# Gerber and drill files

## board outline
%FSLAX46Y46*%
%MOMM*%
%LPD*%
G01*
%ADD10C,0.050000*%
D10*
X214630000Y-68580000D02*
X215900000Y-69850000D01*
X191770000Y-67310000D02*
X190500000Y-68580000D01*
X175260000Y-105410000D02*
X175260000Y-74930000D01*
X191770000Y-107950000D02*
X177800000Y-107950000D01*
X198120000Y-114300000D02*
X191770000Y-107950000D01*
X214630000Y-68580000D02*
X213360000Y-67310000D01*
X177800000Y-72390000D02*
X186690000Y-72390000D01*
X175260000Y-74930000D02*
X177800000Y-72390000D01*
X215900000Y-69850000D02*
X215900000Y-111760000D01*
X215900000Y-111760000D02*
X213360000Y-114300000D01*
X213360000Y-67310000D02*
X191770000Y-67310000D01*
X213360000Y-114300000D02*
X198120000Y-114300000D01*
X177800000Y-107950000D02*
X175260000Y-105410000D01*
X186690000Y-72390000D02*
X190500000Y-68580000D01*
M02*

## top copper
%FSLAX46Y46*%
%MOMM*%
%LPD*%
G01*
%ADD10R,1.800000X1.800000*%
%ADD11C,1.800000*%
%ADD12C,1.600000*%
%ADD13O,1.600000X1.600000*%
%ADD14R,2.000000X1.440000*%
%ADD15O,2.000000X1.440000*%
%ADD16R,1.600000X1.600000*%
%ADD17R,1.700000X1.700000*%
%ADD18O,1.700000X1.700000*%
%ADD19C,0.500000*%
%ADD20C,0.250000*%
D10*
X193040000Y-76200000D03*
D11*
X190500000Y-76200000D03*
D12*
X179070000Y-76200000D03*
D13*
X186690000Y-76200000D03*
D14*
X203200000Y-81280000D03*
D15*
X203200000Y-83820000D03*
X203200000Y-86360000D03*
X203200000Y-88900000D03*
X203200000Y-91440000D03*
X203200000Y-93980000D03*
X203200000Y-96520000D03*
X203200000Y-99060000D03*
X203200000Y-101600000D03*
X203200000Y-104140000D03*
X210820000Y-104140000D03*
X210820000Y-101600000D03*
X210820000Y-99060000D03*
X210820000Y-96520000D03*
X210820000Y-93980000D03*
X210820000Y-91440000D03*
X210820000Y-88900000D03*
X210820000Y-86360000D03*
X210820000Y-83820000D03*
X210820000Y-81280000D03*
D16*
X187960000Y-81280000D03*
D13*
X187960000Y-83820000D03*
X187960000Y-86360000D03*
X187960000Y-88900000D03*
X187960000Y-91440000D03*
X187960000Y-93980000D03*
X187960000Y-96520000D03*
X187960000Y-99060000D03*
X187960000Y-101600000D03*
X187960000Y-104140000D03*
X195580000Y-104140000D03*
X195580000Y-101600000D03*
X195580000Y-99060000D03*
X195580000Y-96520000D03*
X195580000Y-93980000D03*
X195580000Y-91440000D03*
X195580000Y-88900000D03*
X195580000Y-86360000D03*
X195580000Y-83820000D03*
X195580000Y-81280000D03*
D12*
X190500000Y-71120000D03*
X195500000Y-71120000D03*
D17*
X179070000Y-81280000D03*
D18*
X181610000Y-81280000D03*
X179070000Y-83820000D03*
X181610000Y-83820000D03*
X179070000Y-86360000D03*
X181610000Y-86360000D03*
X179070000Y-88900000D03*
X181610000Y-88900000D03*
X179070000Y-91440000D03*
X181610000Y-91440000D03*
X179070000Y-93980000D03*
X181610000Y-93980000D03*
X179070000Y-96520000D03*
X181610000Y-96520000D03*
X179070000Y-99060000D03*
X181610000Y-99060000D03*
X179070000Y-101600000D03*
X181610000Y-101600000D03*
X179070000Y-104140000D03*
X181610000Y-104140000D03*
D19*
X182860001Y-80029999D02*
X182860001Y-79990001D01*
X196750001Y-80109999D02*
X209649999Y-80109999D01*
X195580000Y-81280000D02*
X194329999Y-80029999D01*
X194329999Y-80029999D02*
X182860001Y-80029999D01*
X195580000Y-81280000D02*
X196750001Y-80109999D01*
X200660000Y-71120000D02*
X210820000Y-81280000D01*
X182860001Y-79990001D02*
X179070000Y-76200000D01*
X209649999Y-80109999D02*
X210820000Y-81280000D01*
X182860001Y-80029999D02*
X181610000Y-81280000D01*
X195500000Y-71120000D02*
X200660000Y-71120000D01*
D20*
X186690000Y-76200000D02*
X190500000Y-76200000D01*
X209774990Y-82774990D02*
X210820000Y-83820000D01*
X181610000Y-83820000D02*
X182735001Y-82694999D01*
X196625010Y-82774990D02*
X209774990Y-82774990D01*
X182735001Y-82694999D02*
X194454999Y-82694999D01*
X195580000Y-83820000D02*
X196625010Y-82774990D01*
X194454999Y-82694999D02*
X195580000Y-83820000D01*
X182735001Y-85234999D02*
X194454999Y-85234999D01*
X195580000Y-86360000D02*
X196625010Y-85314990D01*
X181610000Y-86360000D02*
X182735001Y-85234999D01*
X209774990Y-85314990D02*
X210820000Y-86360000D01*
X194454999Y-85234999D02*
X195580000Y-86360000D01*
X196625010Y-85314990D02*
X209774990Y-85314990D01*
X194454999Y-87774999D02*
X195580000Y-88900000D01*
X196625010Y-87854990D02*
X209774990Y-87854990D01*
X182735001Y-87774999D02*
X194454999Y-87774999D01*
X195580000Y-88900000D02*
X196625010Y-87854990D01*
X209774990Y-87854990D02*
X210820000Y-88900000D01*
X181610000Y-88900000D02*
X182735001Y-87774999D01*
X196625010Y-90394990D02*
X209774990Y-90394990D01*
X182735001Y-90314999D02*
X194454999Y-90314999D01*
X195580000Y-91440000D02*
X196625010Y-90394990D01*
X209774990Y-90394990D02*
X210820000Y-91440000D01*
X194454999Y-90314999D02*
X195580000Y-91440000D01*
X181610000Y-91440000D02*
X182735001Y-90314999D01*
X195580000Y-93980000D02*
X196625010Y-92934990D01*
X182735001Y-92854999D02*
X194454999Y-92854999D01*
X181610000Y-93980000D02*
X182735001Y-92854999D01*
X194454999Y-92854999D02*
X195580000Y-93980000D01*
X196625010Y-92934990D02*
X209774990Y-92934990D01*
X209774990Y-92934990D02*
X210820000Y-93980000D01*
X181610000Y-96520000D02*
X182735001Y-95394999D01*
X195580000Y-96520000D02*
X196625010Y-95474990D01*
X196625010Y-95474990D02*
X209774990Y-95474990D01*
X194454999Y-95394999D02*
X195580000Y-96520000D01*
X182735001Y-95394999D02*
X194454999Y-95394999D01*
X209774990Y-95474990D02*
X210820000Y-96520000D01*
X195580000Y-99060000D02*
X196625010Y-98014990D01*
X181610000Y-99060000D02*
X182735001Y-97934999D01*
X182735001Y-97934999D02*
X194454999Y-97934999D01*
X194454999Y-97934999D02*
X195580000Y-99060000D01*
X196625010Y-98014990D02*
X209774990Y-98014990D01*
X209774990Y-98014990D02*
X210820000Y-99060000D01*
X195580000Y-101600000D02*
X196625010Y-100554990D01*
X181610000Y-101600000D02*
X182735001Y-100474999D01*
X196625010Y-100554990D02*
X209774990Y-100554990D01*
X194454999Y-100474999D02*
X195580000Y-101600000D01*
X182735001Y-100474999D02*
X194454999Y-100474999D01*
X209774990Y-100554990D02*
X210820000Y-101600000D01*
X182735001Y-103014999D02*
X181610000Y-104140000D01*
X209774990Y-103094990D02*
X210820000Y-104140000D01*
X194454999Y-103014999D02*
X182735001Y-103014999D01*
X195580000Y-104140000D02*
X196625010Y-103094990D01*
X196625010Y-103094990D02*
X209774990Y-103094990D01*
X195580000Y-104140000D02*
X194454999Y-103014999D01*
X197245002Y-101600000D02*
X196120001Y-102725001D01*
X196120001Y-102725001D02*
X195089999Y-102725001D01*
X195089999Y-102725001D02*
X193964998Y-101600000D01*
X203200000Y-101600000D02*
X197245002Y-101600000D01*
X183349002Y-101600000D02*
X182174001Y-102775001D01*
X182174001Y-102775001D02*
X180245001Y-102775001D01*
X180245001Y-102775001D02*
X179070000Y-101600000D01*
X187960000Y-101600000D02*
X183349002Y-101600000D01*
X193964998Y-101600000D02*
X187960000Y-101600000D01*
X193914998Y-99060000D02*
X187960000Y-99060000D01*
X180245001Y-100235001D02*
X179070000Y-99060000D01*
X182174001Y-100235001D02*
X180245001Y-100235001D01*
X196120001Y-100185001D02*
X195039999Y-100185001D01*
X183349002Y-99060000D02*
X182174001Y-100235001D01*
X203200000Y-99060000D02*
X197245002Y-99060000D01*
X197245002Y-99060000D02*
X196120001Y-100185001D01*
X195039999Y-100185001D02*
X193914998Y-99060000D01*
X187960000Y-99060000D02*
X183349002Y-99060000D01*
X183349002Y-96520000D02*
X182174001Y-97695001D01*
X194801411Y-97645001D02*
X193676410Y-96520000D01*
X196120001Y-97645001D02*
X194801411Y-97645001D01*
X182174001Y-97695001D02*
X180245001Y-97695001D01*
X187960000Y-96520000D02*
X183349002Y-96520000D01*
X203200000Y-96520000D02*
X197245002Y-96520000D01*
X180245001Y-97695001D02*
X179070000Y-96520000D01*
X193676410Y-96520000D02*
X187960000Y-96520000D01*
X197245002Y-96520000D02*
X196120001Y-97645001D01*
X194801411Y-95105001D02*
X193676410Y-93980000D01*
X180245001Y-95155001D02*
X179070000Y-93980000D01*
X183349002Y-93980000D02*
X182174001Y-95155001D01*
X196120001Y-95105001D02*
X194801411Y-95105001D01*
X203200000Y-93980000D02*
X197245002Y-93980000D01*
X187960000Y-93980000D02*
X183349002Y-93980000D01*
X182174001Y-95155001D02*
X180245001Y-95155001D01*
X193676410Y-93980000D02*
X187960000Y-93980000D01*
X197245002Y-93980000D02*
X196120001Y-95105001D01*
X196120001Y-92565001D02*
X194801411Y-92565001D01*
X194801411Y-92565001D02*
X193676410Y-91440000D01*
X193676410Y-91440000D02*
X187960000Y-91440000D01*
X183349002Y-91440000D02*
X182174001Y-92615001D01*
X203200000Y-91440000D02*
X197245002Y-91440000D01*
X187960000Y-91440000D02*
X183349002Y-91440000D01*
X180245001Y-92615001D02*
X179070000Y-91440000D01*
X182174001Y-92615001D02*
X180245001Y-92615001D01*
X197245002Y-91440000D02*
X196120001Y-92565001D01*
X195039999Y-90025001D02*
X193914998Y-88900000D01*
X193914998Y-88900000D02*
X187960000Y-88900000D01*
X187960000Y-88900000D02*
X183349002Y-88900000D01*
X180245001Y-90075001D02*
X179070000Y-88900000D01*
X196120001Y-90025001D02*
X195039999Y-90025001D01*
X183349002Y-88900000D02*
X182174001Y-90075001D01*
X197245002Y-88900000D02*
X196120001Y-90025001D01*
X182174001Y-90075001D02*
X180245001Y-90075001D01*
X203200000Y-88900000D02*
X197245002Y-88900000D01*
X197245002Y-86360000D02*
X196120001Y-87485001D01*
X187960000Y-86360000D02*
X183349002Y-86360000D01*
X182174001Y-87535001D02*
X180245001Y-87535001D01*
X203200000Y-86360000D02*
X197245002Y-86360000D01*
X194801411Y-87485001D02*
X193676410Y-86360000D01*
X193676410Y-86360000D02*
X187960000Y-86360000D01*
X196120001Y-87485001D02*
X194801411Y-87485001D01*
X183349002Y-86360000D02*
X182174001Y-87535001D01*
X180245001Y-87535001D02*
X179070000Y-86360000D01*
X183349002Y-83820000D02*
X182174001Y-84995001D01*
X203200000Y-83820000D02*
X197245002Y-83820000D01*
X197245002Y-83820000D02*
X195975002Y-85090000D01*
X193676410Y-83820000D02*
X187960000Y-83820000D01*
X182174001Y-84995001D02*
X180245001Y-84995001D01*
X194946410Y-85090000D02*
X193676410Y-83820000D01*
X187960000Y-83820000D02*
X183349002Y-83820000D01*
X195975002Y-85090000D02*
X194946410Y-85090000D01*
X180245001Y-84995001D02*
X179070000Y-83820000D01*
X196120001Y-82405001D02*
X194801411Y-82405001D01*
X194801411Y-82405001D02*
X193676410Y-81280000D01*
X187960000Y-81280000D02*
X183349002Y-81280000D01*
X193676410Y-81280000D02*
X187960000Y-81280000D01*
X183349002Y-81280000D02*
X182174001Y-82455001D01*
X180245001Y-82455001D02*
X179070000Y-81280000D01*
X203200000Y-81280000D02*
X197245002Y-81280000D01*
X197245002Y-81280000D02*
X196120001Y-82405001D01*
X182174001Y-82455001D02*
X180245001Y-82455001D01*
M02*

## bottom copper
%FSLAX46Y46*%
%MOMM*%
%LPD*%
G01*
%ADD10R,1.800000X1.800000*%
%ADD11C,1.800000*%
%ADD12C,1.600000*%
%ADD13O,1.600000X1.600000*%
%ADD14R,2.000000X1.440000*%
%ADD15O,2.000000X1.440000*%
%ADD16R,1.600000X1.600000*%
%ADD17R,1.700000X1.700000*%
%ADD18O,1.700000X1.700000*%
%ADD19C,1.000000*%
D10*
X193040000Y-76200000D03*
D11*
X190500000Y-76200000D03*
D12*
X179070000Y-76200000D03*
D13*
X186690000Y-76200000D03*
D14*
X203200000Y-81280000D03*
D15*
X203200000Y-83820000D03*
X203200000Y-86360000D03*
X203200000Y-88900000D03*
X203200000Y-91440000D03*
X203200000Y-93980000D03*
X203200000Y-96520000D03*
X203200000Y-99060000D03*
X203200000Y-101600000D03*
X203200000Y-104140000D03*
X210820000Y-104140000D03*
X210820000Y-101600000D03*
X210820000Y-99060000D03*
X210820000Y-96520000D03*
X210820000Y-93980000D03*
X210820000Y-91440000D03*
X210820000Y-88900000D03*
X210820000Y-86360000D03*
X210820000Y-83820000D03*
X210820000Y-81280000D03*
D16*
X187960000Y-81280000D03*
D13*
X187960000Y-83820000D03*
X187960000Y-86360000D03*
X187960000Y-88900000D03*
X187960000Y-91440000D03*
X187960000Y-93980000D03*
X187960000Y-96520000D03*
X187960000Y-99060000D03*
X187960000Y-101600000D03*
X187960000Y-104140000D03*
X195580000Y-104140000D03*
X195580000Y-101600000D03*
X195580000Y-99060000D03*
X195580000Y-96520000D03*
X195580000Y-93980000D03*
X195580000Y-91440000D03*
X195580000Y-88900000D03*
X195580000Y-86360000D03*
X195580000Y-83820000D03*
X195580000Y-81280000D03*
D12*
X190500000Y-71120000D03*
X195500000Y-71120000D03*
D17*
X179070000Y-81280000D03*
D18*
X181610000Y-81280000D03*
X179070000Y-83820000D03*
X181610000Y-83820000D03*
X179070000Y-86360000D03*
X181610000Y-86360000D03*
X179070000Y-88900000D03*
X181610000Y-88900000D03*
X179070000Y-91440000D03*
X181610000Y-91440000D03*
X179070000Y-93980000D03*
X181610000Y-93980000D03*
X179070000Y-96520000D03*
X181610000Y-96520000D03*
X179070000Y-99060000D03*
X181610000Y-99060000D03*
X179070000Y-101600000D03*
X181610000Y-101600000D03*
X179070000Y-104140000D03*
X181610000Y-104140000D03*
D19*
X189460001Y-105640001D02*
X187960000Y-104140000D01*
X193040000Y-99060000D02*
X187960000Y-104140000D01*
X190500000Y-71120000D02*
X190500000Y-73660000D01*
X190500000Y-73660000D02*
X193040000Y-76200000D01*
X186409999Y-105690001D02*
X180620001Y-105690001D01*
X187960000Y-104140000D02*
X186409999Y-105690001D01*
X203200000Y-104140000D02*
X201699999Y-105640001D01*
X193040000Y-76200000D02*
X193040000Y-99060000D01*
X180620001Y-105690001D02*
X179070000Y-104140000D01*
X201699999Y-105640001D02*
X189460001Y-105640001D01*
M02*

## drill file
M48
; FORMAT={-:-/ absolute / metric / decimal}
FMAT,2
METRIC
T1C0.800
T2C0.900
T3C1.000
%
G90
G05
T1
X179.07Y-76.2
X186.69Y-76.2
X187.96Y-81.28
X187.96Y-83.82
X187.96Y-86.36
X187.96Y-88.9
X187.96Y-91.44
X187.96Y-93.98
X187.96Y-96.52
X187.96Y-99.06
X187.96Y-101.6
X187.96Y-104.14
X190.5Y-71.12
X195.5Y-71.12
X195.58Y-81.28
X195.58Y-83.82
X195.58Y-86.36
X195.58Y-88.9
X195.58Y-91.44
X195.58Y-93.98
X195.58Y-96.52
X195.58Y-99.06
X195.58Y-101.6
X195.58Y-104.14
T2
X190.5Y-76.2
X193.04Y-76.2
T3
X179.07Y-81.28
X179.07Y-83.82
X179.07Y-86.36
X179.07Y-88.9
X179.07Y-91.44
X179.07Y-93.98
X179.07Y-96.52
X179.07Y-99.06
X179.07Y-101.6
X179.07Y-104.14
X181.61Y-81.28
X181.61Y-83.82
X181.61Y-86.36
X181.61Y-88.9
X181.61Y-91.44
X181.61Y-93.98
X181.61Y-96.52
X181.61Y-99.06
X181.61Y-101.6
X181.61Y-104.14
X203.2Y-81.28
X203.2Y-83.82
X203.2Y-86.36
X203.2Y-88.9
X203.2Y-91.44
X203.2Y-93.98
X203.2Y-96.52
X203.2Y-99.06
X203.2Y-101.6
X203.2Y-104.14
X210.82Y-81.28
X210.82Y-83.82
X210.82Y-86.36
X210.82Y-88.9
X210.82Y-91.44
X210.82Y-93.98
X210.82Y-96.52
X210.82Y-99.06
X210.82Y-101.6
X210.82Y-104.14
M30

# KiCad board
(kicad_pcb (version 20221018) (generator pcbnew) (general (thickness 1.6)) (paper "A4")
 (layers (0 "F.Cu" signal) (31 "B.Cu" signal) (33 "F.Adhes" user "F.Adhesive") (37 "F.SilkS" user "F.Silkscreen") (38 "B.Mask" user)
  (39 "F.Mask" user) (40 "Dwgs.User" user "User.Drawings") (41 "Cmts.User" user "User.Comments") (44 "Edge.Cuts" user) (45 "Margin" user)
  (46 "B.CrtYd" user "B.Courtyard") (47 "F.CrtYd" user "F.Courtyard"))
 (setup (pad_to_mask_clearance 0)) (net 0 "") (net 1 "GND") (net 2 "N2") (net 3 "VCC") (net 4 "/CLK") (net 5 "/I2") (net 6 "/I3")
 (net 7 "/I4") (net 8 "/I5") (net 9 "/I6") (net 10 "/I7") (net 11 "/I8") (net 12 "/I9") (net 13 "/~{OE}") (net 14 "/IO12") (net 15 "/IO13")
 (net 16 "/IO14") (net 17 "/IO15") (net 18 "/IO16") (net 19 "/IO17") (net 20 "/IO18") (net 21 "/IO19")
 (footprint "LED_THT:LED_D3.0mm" (layer "F.Cu") (at 193.04 76.2 180)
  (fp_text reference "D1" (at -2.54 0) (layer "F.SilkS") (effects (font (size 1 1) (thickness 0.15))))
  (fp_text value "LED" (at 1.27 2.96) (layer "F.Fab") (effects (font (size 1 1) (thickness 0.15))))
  (pad "1" thru_hole rect (at 0 0 180) (size 1.8 1.8) (drill 0.9) (layers "*.Cu" "*.Mask") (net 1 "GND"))
  (pad "2" thru_hole circle (at 2.54 0 180) (size 1.8 1.8) (drill 0.9) (layers "*.Cu" "*.Mask") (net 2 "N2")))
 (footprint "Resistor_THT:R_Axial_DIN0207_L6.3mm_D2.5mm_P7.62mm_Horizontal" (layer "F.Cu") (at 179.07 76.2)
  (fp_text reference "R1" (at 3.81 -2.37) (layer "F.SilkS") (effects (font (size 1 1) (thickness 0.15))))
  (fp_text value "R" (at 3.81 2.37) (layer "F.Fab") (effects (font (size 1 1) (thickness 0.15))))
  (pad "1" thru_hole circle (at 0 0) (size 1.6 1.6) (drill 0.8) (layers "*.Cu" "*.Mask") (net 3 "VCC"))
  (pad "2" thru_hole oval (at 7.62 0) (size 1.6 1.6) (drill 0.8) (layers "*.Cu" "*.Mask") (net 2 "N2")))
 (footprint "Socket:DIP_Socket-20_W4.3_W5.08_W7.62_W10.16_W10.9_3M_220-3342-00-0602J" (layer "F.Cu") (at 203.2 81.28)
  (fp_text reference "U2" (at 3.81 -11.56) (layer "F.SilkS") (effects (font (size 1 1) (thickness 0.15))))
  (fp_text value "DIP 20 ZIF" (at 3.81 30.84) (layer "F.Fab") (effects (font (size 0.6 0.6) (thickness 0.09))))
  (pad "1" thru_hole rect (at 0 0) (size 2 1.44) (drill 1) (layers "*.Cu" "*.Mask") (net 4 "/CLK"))
  (pad "2" thru_hole oval (at 0 2.54) (size 2 1.44) (drill 1) (layers "*.Cu" "*.Mask") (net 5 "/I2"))
  (pad "3" thru_hole oval (at 0 5.08) (size 2 1.44) (drill 1) (layers "*.Cu" "*.Mask") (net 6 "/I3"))
  (pad "4" thru_hole oval (at 0 7.62) (size 2 1.44) (drill 1) (layers "*.Cu" "*.Mask") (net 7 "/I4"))
  (pad "5" thru_hole oval (at 0 10.16) (size 2 1.44) (drill 1) (layers "*.Cu" "*.Mask") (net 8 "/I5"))
  (pad "6" thru_hole oval (at 0 12.7) (size 2 1.44) (drill 1) (layers "*.Cu" "*.Mask") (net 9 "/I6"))
  (pad "7" thru_hole oval (at 0 15.24) (size 2 1.44) (drill 1) (layers "*.Cu" "*.Mask") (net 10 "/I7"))
  (pad "8" thru_hole oval (at 0 17.78) (size 2 1.44) (drill 1) (layers "*.Cu" "*.Mask") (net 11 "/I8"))
  (pad "9" thru_hole oval (at 0 20.32) (size 2 1.44) (drill 1) (layers "*.Cu" "*.Mask") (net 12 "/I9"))
  (pad "10" thru_hole oval (at 0 22.86) (size 2 1.44) (drill 1) (layers "*.Cu" "*.Mask") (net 1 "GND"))
  (pad "11" thru_hole oval (at 7.62 22.86) (size 2 1.44) (drill 1) (layers "*.Cu" "*.Mask") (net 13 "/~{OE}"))
  (pad "12" thru_hole oval (at 7.62 20.32) (size 2 1.44) (drill 1) (layers "*.Cu" "*.Mask") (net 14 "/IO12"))
  (pad "13" thru_hole oval (at 7.62 17.78) (size 2 1.44) (drill 1) (layers "*.Cu" "*.Mask") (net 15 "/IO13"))
  (pad "14" thru_hole oval (at 7.62 15.24) (size 2 1.44) (drill 1) (layers "*.Cu" "*.Mask") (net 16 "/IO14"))
  (pad "15" thru_hole oval (at 7.62 12.7) (size 2 1.44) (drill 1) (layers "*.Cu" "*.Mask") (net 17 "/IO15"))
  (pad "16" thru_hole oval (at 7.62 10.16) (size 2 1.44) (drill 1) (layers "*.Cu" "*.Mask") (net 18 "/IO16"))
  (pad "17" thru_hole oval (at 7.62 7.62) (size 2 1.44) (drill 1) (layers "*.Cu" "*.Mask") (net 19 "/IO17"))
  (pad "18" thru_hole oval (at 7.62 5.08) (size 2 1.44) (drill 1) (layers "*.Cu" "*.Mask") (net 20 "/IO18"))
  (pad "19" thru_hole oval (at 7.62 2.54) (size 2 1.44) (drill 1) (layers "*.Cu" "*.Mask") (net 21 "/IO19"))
  (pad "20" thru_hole oval (at 7.62 0) (size 2 1.44) (drill 1) (layers "*.Cu" "*.Mask") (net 3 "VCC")))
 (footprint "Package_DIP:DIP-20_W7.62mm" (layer "F.Cu") (at 187.96 81.28)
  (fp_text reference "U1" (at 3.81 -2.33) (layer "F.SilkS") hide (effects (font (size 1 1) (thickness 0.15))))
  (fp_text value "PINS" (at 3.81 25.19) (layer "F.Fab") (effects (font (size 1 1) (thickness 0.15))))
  (pad "1" thru_hole rect (at 0 0) (size 1.6 1.6) (drill 0.8) (layers "*.Cu" "*.Mask") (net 4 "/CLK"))
  (pad "2" thru_hole oval (at 0 2.54) (size 1.6 1.6) (drill 0.8) (layers "*.Cu" "*.Mask") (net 5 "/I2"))
  (pad "3" thru_hole oval (at 0 5.08) (size 1.6 1.6) (drill 0.8) (layers "*.Cu" "*.Mask") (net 6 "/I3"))
  (pad "4" thru_hole oval (at 0 7.62) (size 1.6 1.6) (drill 0.8) (layers "*.Cu" "*.Mask") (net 7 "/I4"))
  (pad "5" thru_hole oval (at 0 10.16) (size 1.6 1.6) (drill 0.8) (layers "*.Cu" "*.Mask") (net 8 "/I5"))
  (pad "6" thru_hole oval (at 0 12.7) (size 1.6 1.6) (drill 0.8) (layers "*.Cu" "*.Mask") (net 9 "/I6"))
  (pad "7" thru_hole oval (at 0 15.24) (size 1.6 1.6) (drill 0.8) (layers "*.Cu" "*.Mask") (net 10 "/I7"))
  (pad "8" thru_hole oval (at 0 17.78) (size 1.6 1.6) (drill 0.8) (layers "*.Cu" "*.Mask") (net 11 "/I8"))
  (pad "9" thru_hole oval (at 0 20.32) (size 1.6 1.6) (drill 0.8) (layers "*.Cu" "*.Mask") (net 12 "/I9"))
  (pad "10" thru_hole oval (at 0 22.86) (size 1.6 1.6) (drill 0.8) (layers "*.Cu" "*.Mask") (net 1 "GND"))
  (pad "11" thru_hole oval (at 7.62 22.86) (size 1.6 1.6) (drill 0.8) (layers "*.Cu" "*.Mask") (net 13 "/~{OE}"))
  (pad "12" thru_hole oval (at 7.62 20.32) (size 1.6 1.6) (drill 0.8) (layers "*.Cu" "*.Mask") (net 14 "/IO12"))
  (pad "13" thru_hole oval (at 7.62 17.78) (size 1.6 1.6) (drill 0.8) (layers "*.Cu" "*.Mask") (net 15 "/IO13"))
  (pad "14" thru_hole oval (at 7.62 15.24) (size 1.6 1.6) (drill 0.8) (layers "*.Cu" "*.Mask") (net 16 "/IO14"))
  (pad "15" thru_hole oval (at 7.62 12.7) (size 1.6 1.6) (drill 0.8) (layers "*.Cu" "*.Mask") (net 17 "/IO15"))
  (pad "16" thru_hole oval (at 7.62 10.16) (size 1.6 1.6) (drill 0.8) (layers "*.Cu" "*.Mask") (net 18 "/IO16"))
  (pad "17" thru_hole oval (at 7.62 7.62) (size 1.6 1.6) (drill 0.8) (layers "*.Cu" "*.Mask") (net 19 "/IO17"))
  (pad "18" thru_hole oval (at 7.62 5.08) (size 1.6 1.6) (drill 0.8) (layers "*.Cu" "*.Mask") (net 20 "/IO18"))
  (pad "19" thru_hole oval (at 7.62 2.54) (size 1.6 1.6) (drill 0.8) (layers "*.Cu" "*.Mask") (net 21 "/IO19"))
  (pad "20" thru_hole oval (at 7.62 0) (size 1.6 1.6) (drill 0.8) (layers "*.Cu" "*.Mask") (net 3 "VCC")))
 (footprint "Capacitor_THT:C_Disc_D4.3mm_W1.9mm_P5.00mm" (layer "F.Cu") (at 190.5 71.12)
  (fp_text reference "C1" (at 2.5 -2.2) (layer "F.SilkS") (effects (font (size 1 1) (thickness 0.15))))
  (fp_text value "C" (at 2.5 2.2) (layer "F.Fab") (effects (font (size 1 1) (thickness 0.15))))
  (pad "1" thru_hole circle (at 0 0) (size 1.6 1.6) (drill 0.8) (layers "*.Cu" "*.Mask") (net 1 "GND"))
  (pad "2" thru_hole circle (at 5 0) (size 1.6 1.6) (drill 0.8) (layers "*.Cu" "*.Mask") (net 3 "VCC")))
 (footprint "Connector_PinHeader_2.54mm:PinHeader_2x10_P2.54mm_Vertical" (layer "F.Cu") (at 179.07 81.28)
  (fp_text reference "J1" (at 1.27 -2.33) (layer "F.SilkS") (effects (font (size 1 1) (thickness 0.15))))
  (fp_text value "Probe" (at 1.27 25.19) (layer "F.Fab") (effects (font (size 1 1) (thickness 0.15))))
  (pad "1" thru_hole rect (at 0 0) (size 1.7 1.7) (drill 1) (layers "*.Cu" "*.Mask") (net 4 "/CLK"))
  (pad "2" thru_hole oval (at 2.54 0) (size 1.7 1.7) (drill 1) (layers "*.Cu" "*.Mask") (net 3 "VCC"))
  (pad "3" thru_hole oval (at 0 2.54) (size 1.7 1.7) (drill 1) (layers "*.Cu" "*.Mask") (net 5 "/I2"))
  (pad "4" thru_hole oval (at 2.54 2.54) (size 1.7 1.7) (drill 1) (layers "*.Cu" "*.Mask") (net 21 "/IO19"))
  (pad "5" thru_hole oval (at 0 5.08) (size 1.7 1.7) (drill 1) (layers "*.Cu" "*.Mask") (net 6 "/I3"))
  (pad "6" thru_hole oval (at 2.54 5.08) (size 1.7 1.7) (drill 1) (layers "*.Cu" "*.Mask") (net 20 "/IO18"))
  (pad "7" thru_hole oval (at 0 7.62) (size 1.7 1.7) (drill 1) (layers "*.Cu" "*.Mask") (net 7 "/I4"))
  (pad "8" thru_hole oval (at 2.54 7.62) (size 1.7 1.7) (drill 1) (layers "*.Cu" "*.Mask") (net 19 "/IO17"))
  (pad "9" thru_hole oval (at 0 10.16) (size 1.7 1.7) (drill 1) (layers "*.Cu" "*.Mask") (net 8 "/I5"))
  (pad "10" thru_hole oval (at 2.54 10.16) (size 1.7 1.7) (drill 1) (layers "*.Cu" "*.Mask") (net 18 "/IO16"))
  (pad "11" thru_hole oval (at 0 12.7) (size 1.7 1.7) (drill 1) (layers "*.Cu" "*.Mask") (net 9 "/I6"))
  (pad "12" thru_hole oval (at 2.54 12.7) (size 1.7 1.7) (drill 1) (layers "*.Cu" "*.Mask") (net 17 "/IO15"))
  (pad "13" thru_hole oval (at 0 15.24) (size 1.7 1.7) (drill 1) (layers "*.Cu" "*.Mask") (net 10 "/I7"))
  (pad "14" thru_hole oval (at 2.54 15.24) (size 1.7 1.7) (drill 1) (layers "*.Cu" "*.Mask") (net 16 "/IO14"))
  (pad "15" thru_hole oval (at 0 17.78) (size 1.7 1.7) (drill 1) (layers "*.Cu" "*.Mask") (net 11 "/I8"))
  (pad "16" thru_hole oval (at 2.54 17.78) (size 1.7 1.7) (drill 1) (layers "*.Cu" "*.Mask") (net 15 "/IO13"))
  (pad "17" thru_hole oval (at 0 20.32) (size 1.7 1.7) (drill 1) (layers "*.Cu" "*.Mask") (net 12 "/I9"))
  (pad "18" thru_hole oval (at 2.54 20.32) (size 1.7 1.7) (drill 1) (layers "*.Cu" "*.Mask") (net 14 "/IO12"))
  (pad "19" thru_hole oval (at 0 22.86) (size 1.7 1.7) (drill 1) (layers "*.Cu" "*.Mask") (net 1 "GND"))
  (pad "20" thru_hole oval (at 2.54 22.86) (size 1.7 1.7) (drill 1) (layers "*.Cu" "*.Mask") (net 13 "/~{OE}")))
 (gr_line (start 214.63 68.58) (end 215.9 69.85) (stroke (width 0.05) (type solid)) (layer "Edge.Cuts"))
 (gr_line (start 191.77 67.31) (end 190.5 68.58) (stroke (width 0.05) (type solid)) (layer "Edge.Cuts"))
 (gr_line (start 175.26 105.41) (end 175.26 74.93) (stroke (width 0.05) (type solid)) (layer "Edge.Cuts"))
 (gr_line (start 191.77 107.95) (end 177.8 107.95) (stroke (width 0.05) (type solid)) (layer "Edge.Cuts"))
 (gr_line (start 198.12 114.3) (end 191.77 107.95) (stroke (width 0.05) (type solid)) (layer "Edge.Cuts"))
 (gr_line (start 214.63 68.58) (end 213.36 67.31) (stroke (width 0.05) (type solid)) (layer "Edge.Cuts"))
 (gr_line (start 177.8 72.39) (end 186.69 72.39) (stroke (width 0.05) (type solid)) (layer "Edge.Cuts"))
 (gr_line (start 175.26 74.93) (end 177.8 72.39) (stroke (width 0.05) (type solid)) (layer "Edge.Cuts"))
 (gr_line (start 215.9 69.85) (end 215.9 111.76) (stroke (width 0.05) (type solid)) (layer "Edge.Cuts"))
 (gr_line (start 215.9 111.76) (end 213.36 114.3) (stroke (width 0.05) (type solid)) (layer "Edge.Cuts"))
 (gr_line (start 213.36 67.31) (end 191.77 67.31) (stroke (width 0.05) (type solid)) (layer "Edge.Cuts"))
 (gr_line (start 213.36 114.3) (end 198.12 114.3) (stroke (width 0.05) (type solid)) (layer "Edge.Cuts"))
 (gr_line (start 177.8 107.95) (end 175.26 105.41) (stroke (width 0.05) (type solid)) (layer "Edge.Cuts"))
 (gr_line (start 186.69 72.39) (end 190.5 68.58) (stroke (width 0.05) (type solid)) (layer "Edge.Cuts"))
 (segment (start 182.860001 80.029999) (end 182.860001 79.990001) (width 0.5) (layer "F.Cu") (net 3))
 (segment (start 196.750001 80.109999) (end 209.649999 80.109999) (width 0.5) (layer "F.Cu") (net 3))
 (segment (start 195.58 81.28) (end 194.329999 80.029999) (width 0.5) (layer "F.Cu") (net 3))
 (segment (start 194.329999 80.029999) (end 182.860001 80.029999) (width 0.5) (layer "F.Cu") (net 3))
 (segment (start 195.58 81.28) (end 196.750001 80.109999) (width 0.5) (layer "F.Cu") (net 3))
 (segment (start 200.66 71.12) (end 210.82 81.28) (width 0.5) (layer "F.Cu") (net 3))
 (segment (start 182.860001 79.990001) (end 179.07 76.2) (width 0.5) (layer "F.Cu") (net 3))
 (segment (start 209.649999 80.109999) (end 210.82 81.28) (width 0.5) (layer "F.Cu") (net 3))
 (segment (start 182.860001 80.029999) (end 181.61 81.28) (width 0.5) (layer "F.Cu") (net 3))
 (segment (start 195.5 71.12) (end 200.66 71.12) (width 0.5) (layer "F.Cu") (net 3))
 (segment (start 189.460001 105.640001) (end 187.96 104.14) (width 1) (layer "B.Cu") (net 1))
 (segment (start 193.04 99.06) (end 187.96 104.14) (width 1) (layer "B.Cu") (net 1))
 (segment (start 190.5 71.12) (end 190.5 73.66) (width 1) (layer "B.Cu") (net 1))
 (segment (start 190.5 73.66) (end 193.04 76.2) (width 1) (layer "B.Cu") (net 1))
 (segment (start 186.409999 105.690001) (end 180.620001 105.690001) (width 1) (layer "B.Cu") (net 1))
 (segment (start 187.96 104.14) (end 186.409999 105.690001) (width 1) (layer "B.Cu") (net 1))
 (segment (start 203.2 104.14) (end 201.699999 105.640001) (width 1) (layer "B.Cu") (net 1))
 (segment (start 193.04 76.2) (end 193.04 99.06) (width 1) (layer "B.Cu") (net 1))
 (segment (start 180.620001 105.690001) (end 179.07 104.14) (width 1) (layer "B.Cu") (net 1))
 (segment (start 201.699999 105.640001) (end 189.460001 105.640001) (width 1) (layer "B.Cu") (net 1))
 (segment (start 186.69 76.2) (end 190.5 76.2) (width 0.25) (layer "F.Cu") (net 2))
 (segment (start 209.77499 82.77499) (end 210.82 83.82) (width 0.25) (layer "F.Cu") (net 21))
 (segment (start 181.61 83.82) (end 182.735001 82.694999) (width 0.25) (layer "F.Cu") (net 21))
 (segment (start 196.62501 82.77499) (end 209.77499 82.77499) (width 0.25) (layer "F.Cu") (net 21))
 (segment (start 182.735001 82.694999) (end 194.454999 82.694999) (width 0.25) (layer "F.Cu") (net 21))
 (segment (start 195.58 83.82) (end 196.62501 82.77499) (width 0.25) (layer "F.Cu") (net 21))
 (segment (start 194.454999 82.694999) (end 195.58 83.82) (width 0.25) (layer "F.Cu") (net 21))
 (segment (start 182.735001 85.234999) (end 194.454999 85.234999) (width 0.25) (layer "F.Cu") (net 20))
 (segment (start 195.58 86.36) (end 196.62501 85.31499) (width 0.25) (layer "F.Cu") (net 20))
 (segment (start 181.61 86.36) (end 182.735001 85.234999) (width 0.25) (layer "F.Cu") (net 20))
 (segment (start 209.77499 85.31499) (end 210.82 86.36) (width 0.25) (layer "F.Cu") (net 20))
 (segment (start 194.454999 85.234999) (end 195.58 86.36) (width 0.25) (layer "F.Cu") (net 20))
 (segment (start 196.62501 85.31499) (end 209.77499 85.31499) (width 0.25) (layer "F.Cu") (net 20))
 (segment (start 194.454999 87.774999) (end 195.58 88.9) (width 0.25) (layer "F.Cu") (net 19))
 (segment (start 196.62501 87.85499) (end 209.77499 87.85499) (width 0.25) (layer "F.Cu") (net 19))
 (segment (start 182.735001 87.774999) (end 194.454999 87.774999) (width 0.25) (layer "F.Cu") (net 19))
 (segment (start 195.58 88.9) (end 196.62501 87.85499) (width 0.25) (layer "F.Cu") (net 19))
 (segment (start 209.77499 87.85499) (end 210.82 88.9) (width 0.25) (layer "F.Cu") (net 19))
 (segment (start 181.61 88.9) (end 182.735001 87.774999) (width 0.25) (layer "F.Cu") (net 19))
 (segment (start 196.62501 90.39499) (end 209.77499 90.39499) (width 0.25) (layer "F.Cu") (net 18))
 (segment (start 182.735001 90.314999) (end 194.454999 90.314999) (width 0.25) (layer "F.Cu") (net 18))
 (segment (start 195.58 91.44) (end 196.62501 90.39499) (width 0.25) (layer "F.Cu") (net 18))
 (segment (start 209.77499 90.39499) (end 210.82 91.44) (width 0.25) (layer "F.Cu") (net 18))
 (segment (start 194.454999 90.314999) (end 195.58 91.44) (width 0.25) (layer "F.Cu") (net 18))
 (segment (start 181.61 91.44) (end 182.735001 90.314999) (width 0.25) (layer "F.Cu") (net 18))
 (segment (start 195.58 93.98) (end 196.62501 92.93499) (width 0.25) (layer "F.Cu") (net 17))
 (segment (start 182.735001 92.854999) (end 194.454999 92.854999) (width 0.25) (layer "F.Cu") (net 17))
 (segment (start 181.61 93.98) (end 182.735001 92.854999) (width 0.25) (layer "F.Cu") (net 17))
 (segment (start 194.454999 92.854999) (end 195.58 93.98) (width 0.25) (layer "F.Cu") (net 17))
 (segment (start 196.62501 92.93499) (end 209.77499 92.93499) (width 0.25) (layer "F.Cu") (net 17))
 (segment (start 209.77499 92.93499) (end 210.82 93.98) (width 0.25) (layer "F.Cu") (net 17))
 (segment (start 181.61 96.52) (end 182.735001 95.394999) (width 0.25) (layer "F.Cu") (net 16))
 (segment (start 195.58 96.52) (end 196.62501 95.47499) (width 0.25) (layer "F.Cu") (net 16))
 (segment (start 196.62501 95.47499) (end 209.77499 95.47499) (width 0.25) (layer "F.Cu") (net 16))
 (segment (start 194.454999 95.394999) (end 195.58 96.52) (width 0.25) (layer "F.Cu") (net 16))
 (segment (start 182.735001 95.394999) (end 194.454999 95.394999) (width 0.25) (layer "F.Cu") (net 16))
 (segment (start 209.77499 95.47499) (end 210.82 96.52) (width 0.25) (layer "F.Cu") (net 16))
 (segment (start 195.58 99.06) (end 196.62501 98.01499) (width 0.25) (layer "F.Cu") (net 15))
 (segment (start 181.61 99.06) (end 182.735001 97.934999) (width 0.25) (layer "F.Cu") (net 15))
 (segment (start 182.735001 97.934999) (end 194.454999 97.934999) (width 0.25) (layer "F.Cu") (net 15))
 (segment (start 194.454999 97.934999) (end 195.58 99.06) (width 0.25) (layer "F.Cu") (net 15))
 (segment (start 196.62501 98.01499) (end 209.77499 98.01499) (width 0.25) (layer "F.Cu") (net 15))
 (segment (start 209.77499 98.01499) (end 210.82 99.06) (width 0.25) (layer "F.Cu") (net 15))
 (segment (start 195.58 101.6) (end 196.62501 100.55499) (width 0.25) (layer "F.Cu") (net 14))
 (segment (start 181.61 101.6) (end 182.735001 100.474999) (width 0.25) (layer "F.Cu") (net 14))
 (segment (start 196.62501 100.55499) (end 209.77499 100.55499) (width 0.25) (layer "F.Cu") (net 14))
 (segment (start 194.454999 100.474999) (end 195.58 101.6) (width 0.25) (layer "F.Cu") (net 14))
 (segment (start 182.735001 100.474999) (end 194.454999 100.474999) (width 0.25) (layer "F.Cu") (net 14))
 (segment (start 209.77499 100.55499) (end 210.82 101.6) (width 0.25) (layer "F.Cu") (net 14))
 (segment (start 182.735001 103.014999) (end 181.61 104.14) (width 0.25) (layer "F.Cu") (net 13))
 (segment (start 209.77499 103.09499) (end 210.82 104.14) (width 0.25) (layer "F.Cu") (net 13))
 (segment (start 194.454999 103.014999) (end 182.735001 103.014999) (width 0.25) (layer "F.Cu") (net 13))
 (segment (start 195.58 104.14) (end 196.62501 103.09499) (width 0.25) (layer "F.Cu") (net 13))
 (segment (start 196.62501 103.09499) (end 209.77499 103.09499) (width 0.25) (layer "F.Cu") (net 13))
 (segment (start 195.58 104.14) (end 194.454999 103.014999) (width 0.25) (layer "F.Cu") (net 13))
 (segment (start 197.245002 101.6) (end 196.120001 102.725001) (width 0.25) (layer "F.Cu") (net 12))
 (segment (start 196.120001 102.725001) (end 195.089999 102.725001) (width 0.25) (layer "F.Cu") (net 12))
 (segment (start 195.089999 102.725001) (end 193.964998 101.6) (width 0.25) (layer "F.Cu") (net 12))
 (segment (start 203.2 101.6) (end 197.245002 101.6) (width 0.25) (layer "F.Cu") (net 12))
 (segment (start 183.349002 101.6) (end 182.174001 102.775001) (width 0.25) (layer "F.Cu") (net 12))
 (segment (start 182.174001 102.775001) (end 180.245001 102.775001) (width 0.25) (layer "F.Cu") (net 12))
 (segment (start 180.245001 102.775001) (end 179.07 101.6) (width 0.25) (layer "F.Cu") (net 12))
 (segment (start 187.96 101.6) (end 183.349002 101.6) (width 0.25) (layer "F.Cu") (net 12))
 (segment (start 193.964998 101.6) (end 187.96 101.6) (width 0.25) (layer "F.Cu") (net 12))
 (segment (start 193.914998 99.06) (end 187.96 99.06) (width 0.25) (layer "F.Cu") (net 11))
 (segment (start 180.245001 100.235001) (end 179.07 99.06) (width 0.25) (layer "F.Cu") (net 11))
 (segment (start 182.174001 100.235001) (end 180.245001 100.235001) (width 0.25) (layer "F.Cu") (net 11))
 (segment (start 196.120001 100.185001) (end 195.039999 100.185001) (width 0.25) (layer "F.Cu") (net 11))
 (segment (start 183.349002 99.06) (end 182.174001 100.235001) (width 0.25) (layer "F.Cu") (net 11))
 (segment (start 203.2 99.06) (end 197.245002 99.06) (width 0.25) (layer "F.Cu") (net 11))
 (segment (start 197.245002 99.06) (end 196.120001 100.185001) (width 0.25) (layer "F.Cu") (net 11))
 (segment (start 195.039999 100.185001) (end 193.914998 99.06) (width 0.25) (layer "F.Cu") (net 11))
 (segment (start 187.96 99.06) (end 183.349002 99.06) (width 0.25) (layer "F.Cu") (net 11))
 (segment (start 183.349002 96.52) (end 182.174001 97.695001) (width 0.25) (layer "F.Cu") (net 10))
 (segment (start 194.801411 97.645001) (end 193.67641 96.52) (width 0.25) (layer "F.Cu") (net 10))
 (segment (start 196.120001 97.645001) (end 194.801411 97.645001) (width 0.25) (layer "F.Cu") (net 10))
 (segment (start 182.174001 97.695001) (end 180.245001 97.695001) (width 0.25) (layer "F.Cu") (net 10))
 (segment (start 187.96 96.52) (end 183.349002 96.52) (width 0.25) (layer "F.Cu") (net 10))
 (segment (start 203.2 96.52) (end 197.245002 96.52) (width 0.25) (layer "F.Cu") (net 10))
 (segment (start 180.245001 97.695001) (end 179.07 96.52) (width 0.25) (layer "F.Cu") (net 10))
 (segment (start 193.67641 96.52) (end 187.96 96.52) (width 0.25) (layer "F.Cu") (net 10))
 (segment (start 197.245002 96.52) (end 196.120001 97.645001) (width 0.25) (layer "F.Cu") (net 10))
 (segment (start 194.801411 95.105001) (end 193.67641 93.98) (width 0.25) (layer "F.Cu") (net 9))
 (segment (start 180.245001 95.155001) (end 179.07 93.98) (width 0.25) (layer "F.Cu") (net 9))
 (segment (start 183.349002 93.98) (end 182.174001 95.155001) (width 0.25) (layer "F.Cu") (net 9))
 (segment (start 196.120001 95.105001) (end 194.801411 95.105001) (width 0.25) (layer "F.Cu") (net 9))
 (segment (start 203.2 93.98) (end 197.245002 93.98) (width 0.25) (layer "F.Cu") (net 9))
 (segment (start 187.96 93.98) (end 183.349002 93.98) (width 0.25) (layer "F.Cu") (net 9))
 (segment (start 182.174001 95.155001) (end 180.245001 95.155001) (width 0.25) (layer "F.Cu") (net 9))
 (segment (start 193.67641 93.98) (end 187.96 93.98) (width 0.25) (layer "F.Cu") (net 9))
 (segment (start 197.245002 93.98) (end 196.120001 95.105001) (width 0.25) (layer "F.Cu") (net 9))
 (segment (start 196.120001 92.565001) (end 194.801411 92.565001) (width 0.25) (layer "F.Cu") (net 8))
 (segment (start 194.801411 92.565001) (end 193.67641 91.44) (width 0.25) (layer "F.Cu") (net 8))
 (segment (start 193.67641 91.44) (end 187.96 91.44) (width 0.25) (layer "F.Cu") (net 8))
 (segment (start 183.349002 91.44) (end 182.174001 92.615001) (width 0.25) (layer "F.Cu") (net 8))
 (segment (start 203.2 91.44) (end 197.245002 91.44) (width 0.25) (layer "F.Cu") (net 8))
 (segment (start 187.96 91.44) (end 183.349002 91.44) (width 0.25) (layer "F.Cu") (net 8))
 (segment (start 180.245001 92.615001) (end 179.07 91.44) (width 0.25) (layer "F.Cu") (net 8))
 (segment (start 182.174001 92.615001) (end 180.245001 92.615001) (width 0.25) (layer "F.Cu") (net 8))
 (segment (start 197.245002 91.44) (end 196.120001 92.565001) (width 0.25) (layer "F.Cu") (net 8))
 (segment (start 195.039999 90.025001) (end 193.914998 88.9) (width 0.25) (layer "F.Cu") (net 7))
 (segment (start 193.914998 88.9) (end 187.96 88.9) (width 0.25) (layer "F.Cu") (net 7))
 (segment (start 187.96 88.9) (end 183.349002 88.9) (width 0.25) (layer "F.Cu") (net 7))
 (segment (start 180.245001 90.075001) (end 179.07 88.9) (width 0.25) (layer "F.Cu") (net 7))
 (segment (start 196.120001 90.025001) (end 195.039999 90.025001) (width 0.25) (layer "F.Cu") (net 7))
 (segment (start 183.349002 88.9) (end 182.174001 90.075001) (width 0.25) (layer "F.Cu") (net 7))
 (segment (start 197.245002 88.9) (end 196.120001 90.025001) (width 0.25) (layer "F.Cu") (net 7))
 (segment (start 182.174001 90.075001) (end 180.245001 90.075001) (width 0.25) (layer "F.Cu") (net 7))
 (segment (start 203.2 88.9) (end 197.245002 88.9) (width 0.25) (layer "F.Cu") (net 7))
 (segment (start 197.245002 86.36) (end 196.120001 87.485001) (width 0.25) (layer "F.Cu") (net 6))
 (segment (start 187.96 86.36) (end 183.349002 86.36) (width 0.25) (layer "F.Cu") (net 6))
 (segment (start 182.174001 87.535001) (end 180.245001 87.535001) (width 0.25) (layer "F.Cu") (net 6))
 (segment (start 203.2 86.36) (end 197.245002 86.36) (width 0.25) (layer "F.Cu") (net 6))
 (segment (start 194.801411 87.485001) (end 193.67641 86.36) (width 0.25) (layer "F.Cu") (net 6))
 (segment (start 193.67641 86.36) (end 187.96 86.36) (width 0.25) (layer "F.Cu") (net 6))
 (segment (start 196.120001 87.485001) (end 194.801411 87.485001) (width 0.25) (layer "F.Cu") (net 6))
 (segment (start 183.349002 86.36) (end 182.174001 87.535001) (width 0.25) (layer "F.Cu") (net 6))
 (segment (start 180.245001 87.535001) (end 179.07 86.36) (width 0.25) (layer "F.Cu") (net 6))
 (segment (start 183.349002 83.82) (end 182.174001 84.995001) (width 0.25) (layer "F.Cu") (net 5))
 (segment (start 203.2 83.82) (end 197.245002 83.82) (width 0.25) (layer "F.Cu") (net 5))
 (segment (start 197.245002 83.82) (end 195.975002 85.09) (width 0.25) (layer "F.Cu") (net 5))
 (segment (start 193.67641 83.82) (end 187.96 83.82) (width 0.25) (layer "F.Cu") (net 5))
 (segment (start 182.174001 84.995001) (end 180.245001 84.995001) (width 0.25) (layer "F.Cu") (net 5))
 (segment (start 194.94641 85.09) (end 193.67641 83.82) (width 0.25) (layer "F.Cu") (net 5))
 (segment (start 187.96 83.82) (end 183.349002 83.82) (width 0.25) (layer "F.Cu") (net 5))
 (segment (start 195.975002 85.09) (end 194.94641 85.09) (width 0.25) (layer "F.Cu") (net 5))
 (segment (start 180.245001 84.995001) (end 179.07 83.82) (width 0.25) (layer "F.Cu") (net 5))
 (segment (start 196.120001 82.405001) (end 194.801411 82.405001) (width 0.25) (layer "F.Cu") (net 4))
 (segment (start 194.801411 82.405001) (end 193.67641 81.28) (width 0.25) (layer "F.Cu") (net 4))
 (segment (start 187.96 81.28) (end 183.349002 81.28) (width 0.25) (layer "F.Cu") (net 4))
 (segment (start 193.67641 81.28) (end 187.96 81.28) (width 0.25) (layer "F.Cu") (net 4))
 (segment (start 183.349002 81.28) (end 182.174001 82.455001) (width 0.25) (layer "F.Cu") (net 4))
 (segment (start 180.245001 82.455001) (end 179.07 81.28) (width 0.25) (layer "F.Cu") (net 4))
 (segment (start 203.2 81.28) (end 197.245002 81.28) (width 0.25) (layer "F.Cu") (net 4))
 (segment (start 197.245002 81.28) (end 196.120001 82.405001) (width 0.25) (layer "F.Cu") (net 4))
 (segment (start 182.174001 82.455001) (end 180.245001 82.455001) (width 0.25) (layer "F.Cu") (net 4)))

